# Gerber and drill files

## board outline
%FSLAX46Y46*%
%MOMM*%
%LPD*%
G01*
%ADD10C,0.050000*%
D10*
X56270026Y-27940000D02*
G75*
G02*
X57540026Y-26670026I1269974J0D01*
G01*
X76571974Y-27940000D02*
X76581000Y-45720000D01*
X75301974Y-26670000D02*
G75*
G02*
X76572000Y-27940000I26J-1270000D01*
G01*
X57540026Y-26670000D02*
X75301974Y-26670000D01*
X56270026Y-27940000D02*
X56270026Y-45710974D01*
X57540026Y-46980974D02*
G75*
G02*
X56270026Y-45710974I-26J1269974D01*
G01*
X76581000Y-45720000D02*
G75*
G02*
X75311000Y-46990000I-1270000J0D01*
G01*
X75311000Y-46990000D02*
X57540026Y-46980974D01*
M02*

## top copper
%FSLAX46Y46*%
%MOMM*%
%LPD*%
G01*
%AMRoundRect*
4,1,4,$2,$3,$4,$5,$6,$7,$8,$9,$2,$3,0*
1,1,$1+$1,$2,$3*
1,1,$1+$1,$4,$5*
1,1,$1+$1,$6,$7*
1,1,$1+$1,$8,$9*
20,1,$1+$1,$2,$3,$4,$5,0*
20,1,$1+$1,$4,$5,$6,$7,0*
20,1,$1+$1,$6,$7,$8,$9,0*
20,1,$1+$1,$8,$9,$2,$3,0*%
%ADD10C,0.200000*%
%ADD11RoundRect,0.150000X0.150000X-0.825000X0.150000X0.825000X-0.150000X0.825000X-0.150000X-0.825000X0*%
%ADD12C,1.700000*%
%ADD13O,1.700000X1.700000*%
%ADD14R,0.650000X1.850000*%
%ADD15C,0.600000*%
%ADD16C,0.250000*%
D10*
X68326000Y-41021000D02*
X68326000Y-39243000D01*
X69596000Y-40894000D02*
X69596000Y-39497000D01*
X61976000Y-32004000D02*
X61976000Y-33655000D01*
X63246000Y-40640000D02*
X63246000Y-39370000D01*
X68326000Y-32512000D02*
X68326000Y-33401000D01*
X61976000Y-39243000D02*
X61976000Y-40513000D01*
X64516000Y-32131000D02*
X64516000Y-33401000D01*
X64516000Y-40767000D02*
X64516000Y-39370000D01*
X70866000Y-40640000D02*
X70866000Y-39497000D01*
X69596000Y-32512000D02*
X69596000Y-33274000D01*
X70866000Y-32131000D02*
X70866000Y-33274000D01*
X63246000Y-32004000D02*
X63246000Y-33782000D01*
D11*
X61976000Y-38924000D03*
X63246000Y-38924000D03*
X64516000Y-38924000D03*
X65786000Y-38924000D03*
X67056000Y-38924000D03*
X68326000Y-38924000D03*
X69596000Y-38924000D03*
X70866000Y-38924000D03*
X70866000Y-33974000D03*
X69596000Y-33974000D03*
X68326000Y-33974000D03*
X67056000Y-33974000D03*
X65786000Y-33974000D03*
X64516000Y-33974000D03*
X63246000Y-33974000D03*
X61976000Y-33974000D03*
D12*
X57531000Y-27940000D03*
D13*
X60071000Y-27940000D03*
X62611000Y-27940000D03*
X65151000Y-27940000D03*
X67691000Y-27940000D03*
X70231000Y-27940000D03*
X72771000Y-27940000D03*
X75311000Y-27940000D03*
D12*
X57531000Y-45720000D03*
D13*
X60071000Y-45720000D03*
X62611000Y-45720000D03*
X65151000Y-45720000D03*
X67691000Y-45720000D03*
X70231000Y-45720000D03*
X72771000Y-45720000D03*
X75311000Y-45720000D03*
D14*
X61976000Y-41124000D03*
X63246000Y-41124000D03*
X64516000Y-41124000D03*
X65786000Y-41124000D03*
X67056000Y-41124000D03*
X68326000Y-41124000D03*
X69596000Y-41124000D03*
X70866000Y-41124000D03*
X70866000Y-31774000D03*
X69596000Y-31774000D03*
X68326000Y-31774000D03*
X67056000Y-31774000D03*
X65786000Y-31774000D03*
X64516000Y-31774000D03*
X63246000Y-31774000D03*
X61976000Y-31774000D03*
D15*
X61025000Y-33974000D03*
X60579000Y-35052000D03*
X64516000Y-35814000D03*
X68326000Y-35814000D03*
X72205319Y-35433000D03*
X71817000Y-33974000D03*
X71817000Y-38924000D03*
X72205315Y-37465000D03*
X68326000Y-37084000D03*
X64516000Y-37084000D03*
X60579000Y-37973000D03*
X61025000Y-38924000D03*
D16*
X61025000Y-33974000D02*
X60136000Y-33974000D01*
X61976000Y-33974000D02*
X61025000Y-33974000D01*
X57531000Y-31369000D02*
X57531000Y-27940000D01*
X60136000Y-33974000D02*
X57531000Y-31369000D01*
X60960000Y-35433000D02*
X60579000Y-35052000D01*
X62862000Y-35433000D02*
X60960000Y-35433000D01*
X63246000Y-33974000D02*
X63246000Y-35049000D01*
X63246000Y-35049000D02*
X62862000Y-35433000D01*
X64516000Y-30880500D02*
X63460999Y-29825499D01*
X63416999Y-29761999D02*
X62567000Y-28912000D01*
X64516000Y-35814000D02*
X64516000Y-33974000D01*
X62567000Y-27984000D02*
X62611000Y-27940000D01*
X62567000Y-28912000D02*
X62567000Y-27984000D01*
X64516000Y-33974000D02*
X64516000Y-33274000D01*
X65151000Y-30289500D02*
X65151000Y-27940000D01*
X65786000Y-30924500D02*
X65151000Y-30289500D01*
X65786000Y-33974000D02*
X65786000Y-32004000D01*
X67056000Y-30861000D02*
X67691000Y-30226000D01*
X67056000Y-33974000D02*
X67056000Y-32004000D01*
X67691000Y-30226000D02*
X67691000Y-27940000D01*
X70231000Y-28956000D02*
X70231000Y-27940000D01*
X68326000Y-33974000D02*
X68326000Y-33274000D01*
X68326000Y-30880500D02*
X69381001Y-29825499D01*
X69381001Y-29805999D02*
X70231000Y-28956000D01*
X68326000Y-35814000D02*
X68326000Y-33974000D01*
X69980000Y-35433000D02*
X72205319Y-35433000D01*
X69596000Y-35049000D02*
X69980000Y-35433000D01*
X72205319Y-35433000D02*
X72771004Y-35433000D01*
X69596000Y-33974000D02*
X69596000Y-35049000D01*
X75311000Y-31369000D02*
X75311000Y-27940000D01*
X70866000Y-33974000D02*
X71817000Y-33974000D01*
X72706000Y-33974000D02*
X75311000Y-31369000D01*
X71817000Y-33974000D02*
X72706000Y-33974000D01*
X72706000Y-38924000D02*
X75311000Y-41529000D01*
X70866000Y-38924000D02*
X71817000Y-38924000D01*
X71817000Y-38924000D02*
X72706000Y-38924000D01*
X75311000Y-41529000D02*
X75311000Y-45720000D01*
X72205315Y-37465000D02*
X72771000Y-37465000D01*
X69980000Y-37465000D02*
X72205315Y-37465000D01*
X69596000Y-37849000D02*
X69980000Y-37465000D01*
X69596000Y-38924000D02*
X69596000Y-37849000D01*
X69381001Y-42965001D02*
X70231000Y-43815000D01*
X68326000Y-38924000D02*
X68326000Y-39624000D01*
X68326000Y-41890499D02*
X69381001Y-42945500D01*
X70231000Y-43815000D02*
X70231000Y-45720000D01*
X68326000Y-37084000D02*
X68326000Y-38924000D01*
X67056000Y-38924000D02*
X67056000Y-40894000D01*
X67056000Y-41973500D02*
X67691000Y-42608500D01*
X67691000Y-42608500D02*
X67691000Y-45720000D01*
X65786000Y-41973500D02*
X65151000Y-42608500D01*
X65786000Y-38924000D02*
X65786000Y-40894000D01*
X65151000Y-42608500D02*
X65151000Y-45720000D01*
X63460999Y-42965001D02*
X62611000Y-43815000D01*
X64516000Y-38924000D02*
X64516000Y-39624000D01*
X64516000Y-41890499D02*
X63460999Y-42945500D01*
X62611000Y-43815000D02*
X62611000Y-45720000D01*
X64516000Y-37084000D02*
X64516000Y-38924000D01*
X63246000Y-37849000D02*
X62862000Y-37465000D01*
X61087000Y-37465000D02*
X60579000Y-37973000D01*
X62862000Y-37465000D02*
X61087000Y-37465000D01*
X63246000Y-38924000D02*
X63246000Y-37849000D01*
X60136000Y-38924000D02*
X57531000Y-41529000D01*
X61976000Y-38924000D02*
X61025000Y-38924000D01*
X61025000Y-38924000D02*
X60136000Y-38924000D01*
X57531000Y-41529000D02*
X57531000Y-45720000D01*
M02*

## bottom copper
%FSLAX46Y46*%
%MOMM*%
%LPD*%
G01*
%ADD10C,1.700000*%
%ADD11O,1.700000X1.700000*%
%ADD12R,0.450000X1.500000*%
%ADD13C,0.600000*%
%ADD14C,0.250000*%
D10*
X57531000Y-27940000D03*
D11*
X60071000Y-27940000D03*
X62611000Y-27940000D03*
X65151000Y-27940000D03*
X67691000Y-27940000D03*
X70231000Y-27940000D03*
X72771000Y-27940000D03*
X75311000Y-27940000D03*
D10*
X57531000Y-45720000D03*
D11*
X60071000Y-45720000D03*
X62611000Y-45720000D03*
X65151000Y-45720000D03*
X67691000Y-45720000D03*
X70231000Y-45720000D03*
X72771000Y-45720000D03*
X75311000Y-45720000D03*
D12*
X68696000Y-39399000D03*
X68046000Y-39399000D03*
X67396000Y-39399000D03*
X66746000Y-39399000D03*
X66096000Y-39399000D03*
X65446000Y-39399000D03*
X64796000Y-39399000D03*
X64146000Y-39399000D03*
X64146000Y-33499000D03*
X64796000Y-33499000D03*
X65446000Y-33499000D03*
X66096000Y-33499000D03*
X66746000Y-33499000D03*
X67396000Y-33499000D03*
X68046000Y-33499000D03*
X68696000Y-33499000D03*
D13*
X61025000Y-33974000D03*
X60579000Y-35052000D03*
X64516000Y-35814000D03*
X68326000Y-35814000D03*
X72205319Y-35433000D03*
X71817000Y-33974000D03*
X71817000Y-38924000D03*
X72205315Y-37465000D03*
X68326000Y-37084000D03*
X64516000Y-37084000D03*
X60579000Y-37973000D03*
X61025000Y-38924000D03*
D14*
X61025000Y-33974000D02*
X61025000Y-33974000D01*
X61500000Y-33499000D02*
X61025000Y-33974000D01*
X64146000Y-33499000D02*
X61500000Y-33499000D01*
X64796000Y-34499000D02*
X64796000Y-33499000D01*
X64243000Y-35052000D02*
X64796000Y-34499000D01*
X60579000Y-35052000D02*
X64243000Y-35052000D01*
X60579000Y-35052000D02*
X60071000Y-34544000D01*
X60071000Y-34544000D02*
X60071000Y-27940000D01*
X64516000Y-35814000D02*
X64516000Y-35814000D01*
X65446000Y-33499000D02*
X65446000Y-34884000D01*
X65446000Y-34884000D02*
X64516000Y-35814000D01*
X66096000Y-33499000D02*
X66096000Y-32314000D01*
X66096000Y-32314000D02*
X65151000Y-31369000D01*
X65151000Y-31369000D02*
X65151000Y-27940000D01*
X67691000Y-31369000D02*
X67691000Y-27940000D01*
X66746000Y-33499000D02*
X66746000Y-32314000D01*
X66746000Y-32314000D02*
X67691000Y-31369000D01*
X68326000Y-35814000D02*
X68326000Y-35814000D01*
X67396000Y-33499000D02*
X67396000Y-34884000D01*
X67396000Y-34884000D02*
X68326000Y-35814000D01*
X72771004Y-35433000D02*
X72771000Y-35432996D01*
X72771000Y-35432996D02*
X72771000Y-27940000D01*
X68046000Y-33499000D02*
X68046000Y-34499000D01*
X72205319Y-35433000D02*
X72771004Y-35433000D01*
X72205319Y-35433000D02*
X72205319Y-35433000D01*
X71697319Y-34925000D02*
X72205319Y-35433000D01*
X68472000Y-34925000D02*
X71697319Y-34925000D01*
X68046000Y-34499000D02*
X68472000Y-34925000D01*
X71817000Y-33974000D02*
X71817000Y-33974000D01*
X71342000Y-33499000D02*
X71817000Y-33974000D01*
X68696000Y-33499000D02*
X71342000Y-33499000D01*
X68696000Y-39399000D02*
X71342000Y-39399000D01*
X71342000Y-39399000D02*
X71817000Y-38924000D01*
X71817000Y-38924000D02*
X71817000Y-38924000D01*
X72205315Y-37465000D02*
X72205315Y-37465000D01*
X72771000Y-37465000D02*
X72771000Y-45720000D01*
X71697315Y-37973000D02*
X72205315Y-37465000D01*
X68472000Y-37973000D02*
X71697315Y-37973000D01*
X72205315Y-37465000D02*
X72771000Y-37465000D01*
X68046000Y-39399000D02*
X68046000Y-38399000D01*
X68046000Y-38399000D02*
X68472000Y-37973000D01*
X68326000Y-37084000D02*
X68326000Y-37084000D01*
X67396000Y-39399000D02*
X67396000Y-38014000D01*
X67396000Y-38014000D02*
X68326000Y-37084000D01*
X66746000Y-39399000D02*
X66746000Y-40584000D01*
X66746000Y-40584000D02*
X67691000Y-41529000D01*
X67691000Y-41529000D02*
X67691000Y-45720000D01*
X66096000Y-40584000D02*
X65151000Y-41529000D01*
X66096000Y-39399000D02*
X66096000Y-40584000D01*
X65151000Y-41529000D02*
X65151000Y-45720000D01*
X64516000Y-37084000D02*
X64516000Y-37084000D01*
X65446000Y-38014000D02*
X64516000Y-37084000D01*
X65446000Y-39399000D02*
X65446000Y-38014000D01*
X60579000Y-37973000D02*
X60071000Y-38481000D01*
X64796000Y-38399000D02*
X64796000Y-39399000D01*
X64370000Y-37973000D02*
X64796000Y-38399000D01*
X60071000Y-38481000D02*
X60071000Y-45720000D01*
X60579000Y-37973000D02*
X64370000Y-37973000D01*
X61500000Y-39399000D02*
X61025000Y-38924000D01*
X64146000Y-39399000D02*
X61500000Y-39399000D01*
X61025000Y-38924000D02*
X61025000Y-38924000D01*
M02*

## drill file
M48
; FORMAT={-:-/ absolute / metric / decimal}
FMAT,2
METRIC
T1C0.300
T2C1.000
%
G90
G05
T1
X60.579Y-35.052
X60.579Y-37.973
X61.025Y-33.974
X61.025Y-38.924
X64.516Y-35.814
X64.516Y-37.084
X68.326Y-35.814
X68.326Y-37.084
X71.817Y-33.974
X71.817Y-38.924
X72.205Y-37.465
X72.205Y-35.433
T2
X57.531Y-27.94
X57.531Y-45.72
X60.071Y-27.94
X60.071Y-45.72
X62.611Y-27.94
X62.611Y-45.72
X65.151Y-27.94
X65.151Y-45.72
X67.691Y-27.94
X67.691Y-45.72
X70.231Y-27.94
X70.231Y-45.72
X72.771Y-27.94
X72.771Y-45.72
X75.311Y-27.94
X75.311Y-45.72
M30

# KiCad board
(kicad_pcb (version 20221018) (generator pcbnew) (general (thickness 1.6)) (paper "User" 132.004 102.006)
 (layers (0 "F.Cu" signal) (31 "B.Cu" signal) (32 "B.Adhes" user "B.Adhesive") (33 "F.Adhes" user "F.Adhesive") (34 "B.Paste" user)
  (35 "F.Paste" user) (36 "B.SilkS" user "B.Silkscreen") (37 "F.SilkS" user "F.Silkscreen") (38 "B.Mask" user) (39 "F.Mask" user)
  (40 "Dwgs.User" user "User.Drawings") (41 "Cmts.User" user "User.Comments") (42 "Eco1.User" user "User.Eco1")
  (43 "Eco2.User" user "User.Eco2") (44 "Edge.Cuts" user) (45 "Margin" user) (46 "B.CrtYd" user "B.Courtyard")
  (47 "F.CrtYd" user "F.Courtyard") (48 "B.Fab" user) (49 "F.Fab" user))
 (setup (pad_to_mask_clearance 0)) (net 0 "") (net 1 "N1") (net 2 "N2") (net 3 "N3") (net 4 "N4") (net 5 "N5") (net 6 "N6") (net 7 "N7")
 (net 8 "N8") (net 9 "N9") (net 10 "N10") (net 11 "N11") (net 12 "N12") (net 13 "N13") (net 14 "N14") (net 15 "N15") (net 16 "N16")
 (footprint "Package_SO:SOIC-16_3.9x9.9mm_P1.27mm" (layer "F.Cu") (at 66.421 36.449 90)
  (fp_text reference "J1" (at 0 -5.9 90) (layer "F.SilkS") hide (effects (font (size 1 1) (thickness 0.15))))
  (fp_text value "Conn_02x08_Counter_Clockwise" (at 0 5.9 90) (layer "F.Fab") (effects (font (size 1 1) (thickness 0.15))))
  (pad "1" smd roundrect (at -2.475 -4.445 90) (size 1.95 0.6) (layers "F.Cu" "F.Paste" "F.Mask") (roundrect_rratio 0.25) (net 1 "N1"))
  (pad "2" smd roundrect (at -2.475 -3.175 90) (size 1.95 0.6) (layers "F.Cu" "F.Paste" "F.Mask") (roundrect_rratio 0.25) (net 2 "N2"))
  (pad "3" smd roundrect (at -2.475 -1.905 90) (size 1.95 0.6) (layers "F.Cu" "F.Paste" "F.Mask") (roundrect_rratio 0.25) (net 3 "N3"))
  (pad "4" smd roundrect (at -2.475 -0.635 90) (size 1.95 0.6) (layers "F.Cu" "F.Paste" "F.Mask") (roundrect_rratio 0.25) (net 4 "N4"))
  (pad "5" smd roundrect (at -2.475 0.635 90) (size 1.95 0.6) (layers "F.Cu" "F.Paste" "F.Mask") (roundrect_rratio 0.25) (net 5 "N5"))
  (pad "6" smd roundrect (at -2.475 1.905 90) (size 1.95 0.6) (layers "F.Cu" "F.Paste" "F.Mask") (roundrect_rratio 0.25) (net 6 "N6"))
  (pad "7" smd roundrect (at -2.475 3.175 90) (size 1.95 0.6) (layers "F.Cu" "F.Paste" "F.Mask") (roundrect_rratio 0.25) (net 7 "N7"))
  (pad "8" smd roundrect (at -2.475 4.445 90) (size 1.95 0.6) (layers "F.Cu" "F.Paste" "F.Mask") (roundrect_rratio 0.25) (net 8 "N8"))
  (pad "9" smd roundrect (at 2.475 4.445 90) (size 1.95 0.6) (layers "F.Cu" "F.Paste" "F.Mask") (roundrect_rratio 0.25) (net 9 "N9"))
  (pad "10" smd roundrect (at 2.475 3.175 90) (size 1.95 0.6) (layers "F.Cu" "F.Paste" "F.Mask") (roundrect_rratio 0.25) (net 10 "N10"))
  (pad "11" smd roundrect (at 2.475 1.905 90) (size 1.95 0.6) (layers "F.Cu" "F.Paste" "F.Mask") (roundrect_rratio 0.25) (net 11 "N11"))
  (pad "12" smd roundrect (at 2.475 0.635 90) (size 1.95 0.6) (layers "F.Cu" "F.Paste" "F.Mask") (roundrect_rratio 0.25) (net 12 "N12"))
  (pad "13" smd roundrect (at 2.475 -0.635 90) (size 1.95 0.6) (layers "F.Cu" "F.Paste" "F.Mask") (roundrect_rratio 0.25) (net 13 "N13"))
  (pad "14" smd roundrect (at 2.475 -1.905 90) (size 1.95 0.6) (layers "F.Cu" "F.Paste" "F.Mask") (roundrect_rratio 0.25) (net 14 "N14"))
  (pad "15" smd roundrect (at 2.475 -3.175 90) (size 1.95 0.6) (layers "F.Cu" "F.Paste" "F.Mask") (roundrect_rratio 0.25) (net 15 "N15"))
  (pad "16" smd roundrect (at 2.475 -4.445 90) (size 1.95 0.6) (layers "F.Cu" "F.Paste" "F.Mask") (roundrect_rratio 0.25) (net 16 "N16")))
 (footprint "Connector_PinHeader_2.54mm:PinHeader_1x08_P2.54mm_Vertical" (layer "F.Cu") (at 57.531 27.94 90)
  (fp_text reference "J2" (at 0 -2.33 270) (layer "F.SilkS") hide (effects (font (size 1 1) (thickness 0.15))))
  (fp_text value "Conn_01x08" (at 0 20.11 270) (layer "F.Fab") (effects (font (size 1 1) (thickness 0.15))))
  (pad "1" thru_hole circle (at 0 0 90) (size 1.7 1.7) (drill 1) (layers "*.Cu" "*.Mask") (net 16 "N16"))
  (pad "2" thru_hole oval (at 0 2.54 90) (size 1.7 1.7) (drill 1) (layers "*.Cu" "*.Mask") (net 15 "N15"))
  (pad "3" thru_hole oval (at 0 5.08 90) (size 1.7 1.7) (drill 1) (layers "*.Cu" "*.Mask") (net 14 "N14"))
  (pad "4" thru_hole oval (at 0 7.62 90) (size 1.7 1.7) (drill 1) (layers "*.Cu" "*.Mask") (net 13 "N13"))
  (pad "5" thru_hole oval (at 0 10.16 90) (size 1.7 1.7) (drill 1) (layers "*.Cu" "*.Mask") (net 12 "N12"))
  (pad "6" thru_hole oval (at 0 12.7 90) (size 1.7 1.7) (drill 1) (layers "*.Cu" "*.Mask") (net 11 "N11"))
  (pad "7" thru_hole oval (at 0 15.24 90) (size 1.7 1.7) (drill 1) (layers "*.Cu" "*.Mask") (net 10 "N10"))
  (pad "8" thru_hole oval (at 0 17.78 90) (size 1.7 1.7) (drill 1) (layers "*.Cu" "*.Mask") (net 9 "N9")))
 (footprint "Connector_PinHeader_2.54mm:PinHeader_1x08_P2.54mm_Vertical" (layer "F.Cu") (at 57.531 45.72 90)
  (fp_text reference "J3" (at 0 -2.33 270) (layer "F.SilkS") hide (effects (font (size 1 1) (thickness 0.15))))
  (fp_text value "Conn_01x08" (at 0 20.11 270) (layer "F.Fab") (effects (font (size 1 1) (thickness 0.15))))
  (pad "1" thru_hole circle (at 0 0 90) (size 1.7 1.7) (drill 1) (layers "*.Cu" "*.Mask") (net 1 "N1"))
  (pad "2" thru_hole oval (at 0 2.54 90) (size 1.7 1.7) (drill 1) (layers "*.Cu" "*.Mask") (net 2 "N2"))
  (pad "3" thru_hole oval (at 0 5.08 90) (size 1.7 1.7) (drill 1) (layers "*.Cu" "*.Mask") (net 3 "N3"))
  (pad "4" thru_hole oval (at 0 7.62 90) (size 1.7 1.7) (drill 1) (layers "*.Cu" "*.Mask") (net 4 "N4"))
  (pad "5" thru_hole oval (at 0 10.16 90) (size 1.7 1.7) (drill 1) (layers "*.Cu" "*.Mask") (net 5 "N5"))
  (pad "6" thru_hole oval (at 0 12.7 90) (size 1.7 1.7) (drill 1) (layers "*.Cu" "*.Mask") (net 6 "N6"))
  (pad "7" thru_hole oval (at 0 15.24 90) (size 1.7 1.7) (drill 1) (layers "*.Cu" "*.Mask") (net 7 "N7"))
  (pad "8" thru_hole oval (at 0 17.78 90) (size 1.7 1.7) (drill 1) (layers "*.Cu" "*.Mask") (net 8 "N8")))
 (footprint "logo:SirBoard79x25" (layer "F.Cu") (at 66.421 36.449)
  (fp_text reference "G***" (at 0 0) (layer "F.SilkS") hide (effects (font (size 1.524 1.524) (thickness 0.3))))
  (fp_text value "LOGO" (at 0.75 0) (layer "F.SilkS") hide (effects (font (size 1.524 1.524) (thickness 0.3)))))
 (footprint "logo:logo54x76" (layer "F.Cu") (at 58.801 36.449)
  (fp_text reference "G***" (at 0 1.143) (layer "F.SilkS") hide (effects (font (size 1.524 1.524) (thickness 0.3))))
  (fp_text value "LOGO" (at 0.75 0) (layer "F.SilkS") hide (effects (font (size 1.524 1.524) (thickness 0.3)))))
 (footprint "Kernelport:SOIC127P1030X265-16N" (layer "F.Cu") (at 66.421 36.449 90)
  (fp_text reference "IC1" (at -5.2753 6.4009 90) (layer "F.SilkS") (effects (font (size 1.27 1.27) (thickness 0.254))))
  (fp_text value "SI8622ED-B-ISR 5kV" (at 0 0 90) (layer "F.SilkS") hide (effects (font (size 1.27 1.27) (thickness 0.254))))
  (pad "1" smd rect (at -4.675 -4.445 180) (size 0.65 1.85) (layers "F.Cu" "F.Paste" "F.Mask"))
  (pad "2" smd rect (at -4.675 -3.175 180) (size 0.65 1.85) (layers "F.Cu" "F.Paste" "F.Mask"))
  (pad "3" smd rect (at -4.675 -1.905 180) (size 0.65 1.85) (layers "F.Cu" "F.Paste" "F.Mask"))
  (pad "4" smd rect (at -4.675 -0.635 180) (size 0.65 1.85) (layers "F.Cu" "F.Paste" "F.Mask"))
  (pad "5" smd rect (at -4.675 0.635 180) (size 0.65 1.85) (layers "F.Cu" "F.Paste" "F.Mask"))
  (pad "6" smd rect (at -4.675 1.905 180) (size 0.65 1.85) (layers "F.Cu" "F.Paste" "F.Mask"))
  (pad "7" smd rect (at -4.675 3.175 180) (size 0.65 1.85) (layers "F.Cu" "F.Paste" "F.Mask"))
  (pad "8" smd rect (at -4.675 4.445 180) (size 0.65 1.85) (layers "F.Cu" "F.Paste" "F.Mask"))
  (pad "9" smd rect (at 4.675 4.445 180) (size 0.65 1.85) (layers "F.Cu" "F.Paste" "F.Mask"))
  (pad "10" smd rect (at 4.675 3.175 180) (size 0.65 1.85) (layers "F.Cu" "F.Paste" "F.Mask"))
  (pad "11" smd rect (at 4.675 1.905 180) (size 0.65 1.85) (layers "F.Cu" "F.Paste" "F.Mask"))
  (pad "12" smd rect (at 4.675 0.635 180) (size 0.65 1.85) (layers "F.Cu" "F.Paste" "F.Mask"))
  (pad "13" smd rect (at 4.675 -0.635 180) (size 0.65 1.85) (layers "F.Cu" "F.Paste" "F.Mask"))
  (pad "14" smd rect (at 4.675 -1.905 180) (size 0.65 1.85) (layers "F.Cu" "F.Paste" "F.Mask"))
  (pad "15" smd rect (at 4.675 -3.175 180) (size 0.65 1.85) (layers "F.Cu" "F.Paste" "F.Mask"))
  (pad "16" smd rect (at 4.675 -4.445 180) (size 0.65 1.85) (layers "F.Cu" "F.Paste" "F.Mask")))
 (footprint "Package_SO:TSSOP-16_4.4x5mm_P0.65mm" (layer "B.Cu") (at 66.421 36.449 90)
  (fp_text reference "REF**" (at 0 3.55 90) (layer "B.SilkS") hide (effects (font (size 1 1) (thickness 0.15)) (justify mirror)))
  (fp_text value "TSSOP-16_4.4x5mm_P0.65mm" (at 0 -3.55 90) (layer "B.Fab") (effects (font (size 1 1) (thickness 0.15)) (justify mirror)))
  (pad "1" smd rect (at -2.95 2.275 90) (size 1.5 0.45) (layers "B.Cu" "B.Paste" "B.Mask") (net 8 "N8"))
  (pad "2" smd rect (at -2.95 1.625 90) (size 1.5 0.45) (layers "B.Cu" "B.Paste" "B.Mask") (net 7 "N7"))
  (pad "3" smd rect (at -2.95 0.975 90) (size 1.5 0.45) (layers "B.Cu" "B.Paste" "B.Mask") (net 6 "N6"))
  (pad "4" smd rect (at -2.95 0.325 90) (size 1.5 0.45) (layers "B.Cu" "B.Paste" "B.Mask") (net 5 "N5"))
  (pad "5" smd rect (at -2.95 -0.325 90) (size 1.5 0.45) (layers "B.Cu" "B.Paste" "B.Mask") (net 4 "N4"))
  (pad "6" smd rect (at -2.95 -0.975 90) (size 1.5 0.45) (layers "B.Cu" "B.Paste" "B.Mask") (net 3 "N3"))
  (pad "7" smd rect (at -2.95 -1.625 90) (size 1.5 0.45) (layers "B.Cu" "B.Paste" "B.Mask") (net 2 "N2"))
  (pad "8" smd rect (at -2.95 -2.275 90) (size 1.5 0.45) (layers "B.Cu" "B.Paste" "B.Mask") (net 1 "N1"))
  (pad "9" smd rect (at 2.95 -2.275 90) (size 1.5 0.45) (layers "B.Cu" "B.Paste" "B.Mask") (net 16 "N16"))
  (pad "10" smd rect (at 2.95 -1.625 90) (size 1.5 0.45) (layers "B.Cu" "B.Paste" "B.Mask") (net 15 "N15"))
  (pad "11" smd rect (at 2.95 -0.975 90) (size 1.5 0.45) (layers "B.Cu" "B.Paste" "B.Mask") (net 14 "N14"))
  (pad "12" smd rect (at 2.95 -0.325 90) (size 1.5 0.45) (layers "B.Cu" "B.Paste" "B.Mask") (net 13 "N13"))
  (pad "13" smd rect (at 2.95 0.325 90) (size 1.5 0.45) (layers "B.Cu" "B.Paste" "B.Mask") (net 12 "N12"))
  (pad "14" smd rect (at 2.95 0.975 90) (size 1.5 0.45) (layers "B.Cu" "B.Paste" "B.Mask") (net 11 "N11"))
  (pad "15" smd rect (at 2.95 1.625 90) (size 1.5 0.45) (layers "B.Cu" "B.Paste" "B.Mask") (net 10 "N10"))
  (pad "16" smd rect (at 2.95 2.275 90) (size 1.5 0.45) (layers "B.Cu" "B.Paste" "B.Mask") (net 9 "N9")))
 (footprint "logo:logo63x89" (layer "B.Cu") (at 72.771 36.449 180)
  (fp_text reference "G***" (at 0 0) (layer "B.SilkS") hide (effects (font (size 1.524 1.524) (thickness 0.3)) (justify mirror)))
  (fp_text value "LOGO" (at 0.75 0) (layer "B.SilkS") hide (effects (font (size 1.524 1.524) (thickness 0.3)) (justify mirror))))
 (gr_line (start 68.326 41.021) (end 68.326 39.243) (stroke (width 0.2) (type default)) (layer "F.Cu"))
 (gr_line (start 69.596 40.894) (end 69.596 39.497) (stroke (width 0.2) (type default)) (layer "F.Cu"))
 (gr_line (start 61.976 32.004) (end 61.976 33.655) (stroke (width 0.2) (type default)) (layer "F.Cu"))
 (gr_line (start 63.246 40.64) (end 63.246 39.37) (stroke (width 0.2) (type default)) (layer "F.Cu"))
 (gr_line (start 68.326 32.512) (end 68.326 33.401) (stroke (width 0.2) (type default)) (layer "F.Cu"))
 (gr_line (start 61.976 39.243) (end 61.976 40.513) (stroke (width 0.2) (type default)) (layer "F.Cu"))
 (gr_line (start 64.516 32.131) (end 64.516 33.401) (stroke (width 0.2) (type default)) (layer "F.Cu"))
 (gr_line (start 64.516 40.767) (end 64.516 39.37) (stroke (width 0.2) (type default)) (layer "F.Cu"))
 (gr_line (start 70.866 40.64) (end 70.866 39.497) (stroke (width 0.2) (type default)) (layer "F.Cu"))
 (gr_line (start 69.596 32.512) (end 69.596 33.274) (stroke (width 0.2) (type default)) (layer "F.Cu"))
 (gr_line (start 70.866 32.131) (end 70.866 33.274) (stroke (width 0.2) (type default)) (layer "F.Cu"))
 (gr_line (start 63.246 32.004) (end 63.246 33.782) (stroke (width 0.2) (type default)) (layer "F.Cu"))
 (gr_arc (start 56.270026 27.94) (mid 56.642 27.041974) (end 57.540026 26.67) (stroke (width 0.05) (type default)) (layer "Edge.Cuts"))
 (gr_line (start 76.571974 27.94) (end 76.581 45.72) (stroke (width 0.05) (type default)) (layer "Edge.Cuts"))
 (gr_arc (start 75.301974 26.67) (mid 76.2 27.041974) (end 76.571974 27.94) (stroke (width 0.05) (type default)) (layer "Edge.Cuts"))
 (gr_line (start 57.540026 26.67) (end 75.301974 26.67) (stroke (width 0.05) (type default)) (layer "Edge.Cuts"))
 (gr_line (start 56.270026 27.94) (end 56.270026 45.710974) (stroke (width 0.05) (type default)) (layer "Edge.Cuts"))
 (gr_arc (start 57.540026 46.980974) (mid 56.642 46.609) (end 56.270026 45.710974) (stroke (width 0.05) (type default)) (layer "Edge.Cuts"))
 (gr_arc (start 76.581 45.72) (mid 76.209026 46.618026) (end 75.311 46.99) (stroke (width 0.05) (type default)) (layer "Edge.Cuts"))
 (gr_line (start 75.311 46.99) (end 57.540026 46.980974) (stroke (width 0.05) (type default)) (layer "Edge.Cuts"))
 (segment (start 61.025 33.974) (end 60.136 33.974) (width 0.25) (layer "F.Cu") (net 16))
 (segment (start 61.976 33.974) (end 61.025 33.974) (width 0.25) (layer "F.Cu") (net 16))
 (segment (start 57.531 31.369) (end 57.531 27.94) (width 0.25) (layer "F.Cu") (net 16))
 (segment (start 60.136 33.974) (end 57.531 31.369) (width 0.25) (layer "F.Cu") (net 16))
 (via (at 61.025 33.974) (size 0.6) (drill 0.3) (layers "F.Cu" "B.Cu") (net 16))
 (segment (start 61.025 33.974) (end 61.025 33.974) (width 0.25) (layer "B.Cu") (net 16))
 (segment (start 61.5 33.499) (end 61.025 33.974) (width 0.25) (layer "B.Cu") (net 16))
 (segment (start 64.146 33.499) (end 61.5 33.499) (width 0.25) (layer "B.Cu") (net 16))
 (segment (start 60.96 35.433) (end 60.579 35.052) (width 0.25) (layer "F.Cu") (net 15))
 (segment (start 62.862 35.433) (end 60.96 35.433) (width 0.25) (layer "F.Cu") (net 15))
 (segment (start 63.246 33.974) (end 63.246 35.049) (width 0.25) (layer "F.Cu") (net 15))
 (segment (start 63.246 35.049) (end 62.862 35.433) (width 0.25) (layer "F.Cu") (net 15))
 (via (at 60.579 35.052) (size 0.6) (drill 0.3) (layers "F.Cu" "B.Cu") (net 15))
 (segment (start 64.796 34.499) (end 64.796 33.499) (width 0.25) (layer "B.Cu") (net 15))
 (segment (start 64.243 35.052) (end 64.796 34.499) (width 0.25) (layer "B.Cu") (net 15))
 (segment (start 60.579 35.052) (end 64.243 35.052) (width 0.25) (layer "B.Cu") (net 15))
 (segment (start 60.579 35.052) (end 60.071 34.544) (width 0.25) (layer "B.Cu") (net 15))
 (segment (start 60.071 34.544) (end 60.071 27.94) (width 0.25) (layer "B.Cu") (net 15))
 (segment (start 64.516 30.8805) (end 63.460999 29.825499) (width 0.25) (layer "F.Cu") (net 14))
 (segment (start 63.416999 29.761999) (end 62.567 28.912) (width 0.25) (layer "F.Cu") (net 14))
 (segment (start 64.516 35.814) (end 64.516 33.974) (width 0.25) (layer "F.Cu") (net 14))
 (segment (start 62.567 27.984) (end 62.611 27.94) (width 0.25) (layer "F.Cu") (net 14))
 (segment (start 62.567 28.912) (end 62.567 27.984) (width 0.25) (layer "F.Cu") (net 14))
 (segment (start 64.516 33.974) (end 64.516 33.274) (width 0.25) (layer "F.Cu") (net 14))
 (via (at 64.516 35.814) (size 0.6) (drill 0.3) (layers "F.Cu" "B.Cu") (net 14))
 (segment (start 64.516 35.814) (end 64.516 35.814) (width 0.25) (layer "B.Cu") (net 14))
 (segment (start 65.446 33.499) (end 65.446 34.884) (width 0.25) (layer "B.Cu") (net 14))
 (segment (start 65.446 34.884) (end 64.516 35.814) (width 0.25) (layer "B.Cu") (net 14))
 (segment (start 65.151 30.2895) (end 65.151 27.94) (width 0.25) (layer "F.Cu") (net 13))
 (segment (start 65.786 30.9245) (end 65.151 30.2895) (width 0.25) (layer "F.Cu") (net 13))
 (segment (start 65.786 33.974) (end 65.786 32.004) (width 0.25) (layer "F.Cu") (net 13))
 (segment (start 66.096 33.499) (end 66.096 32.314) (width 0.25) (layer "B.Cu") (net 13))
 (segment (start 66.096 32.314) (end 65.151 31.369) (width 0.25) (layer "B.Cu") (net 13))
 (segment (start 65.151 31.369) (end 65.151 27.94) (width 0.25) (layer "B.Cu") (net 13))
 (segment (start 67.056 30.861) (end 67.691 30.226) (width 0.25) (layer "F.Cu") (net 12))
 (segment (start 67.056 33.974) (end 67.056 32.004) (width 0.25) (layer "F.Cu") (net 12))
 (segment (start 67.691 30.226) (end 67.691 27.94) (width 0.25) (layer "F.Cu") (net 12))
 (segment (start 67.691 31.369) (end 67.691 27.94) (width 0.25) (layer "B.Cu") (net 12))
 (segment (start 66.746 33.499) (end 66.746 32.314) (width 0.25) (layer "B.Cu") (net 12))
 (segment (start 66.746 32.314) (end 67.691 31.369) (width 0.25) (layer "B.Cu") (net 12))
 (segment (start 70.231 28.956) (end 70.231 27.94) (width 0.25) (layer "F.Cu") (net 11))
 (segment (start 68.326 33.974) (end 68.326 33.274) (width 0.25) (layer "F.Cu") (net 11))
 (segment (start 68.326 30.8805) (end 69.381001 29.825499) (width 0.25) (layer "F.Cu") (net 11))
 (segment (start 69.381001 29.805999) (end 70.231 28.956) (width 0.25) (layer "F.Cu") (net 11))
 (segment (start 68.326 35.814) (end 68.326 33.974) (width 0.25) (layer "F.Cu") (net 11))
 (via (at 68.326 35.814) (size 0.6) (drill 0.3) (layers "F.Cu" "B.Cu") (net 11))
 (segment (start 68.326 35.814) (end 68.326 35.814) (width 0.25) (layer "B.Cu") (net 11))
 (segment (start 67.396 33.499) (end 67.396 34.884) (width 0.25) (layer "B.Cu") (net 11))
 (segment (start 67.396 34.884) (end 68.326 35.814) (width 0.25) (layer "B.Cu") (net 11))
 (segment (start 69.98 35.433) (end 72.205319 35.433) (width 0.25) (layer "F.Cu") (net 10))
 (segment (start 69.596 35.049) (end 69.98 35.433) (width 0.25) (layer "F.Cu") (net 10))
 (segment (start 72.205319 35.433) (end 72.771004 35.433) (width 0.25) (layer "F.Cu") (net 10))
 (segment (start 69.596 33.974) (end 69.596 35.049) (width 0.25) (layer "F.Cu") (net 10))
 (via (at 72.205319 35.433) (size 0.6) (drill 0.3) (layers "F.Cu" "B.Cu") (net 10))
 (segment (start 72.771004 35.433) (end 72.771 35.432996) (width 0.25) (layer "B.Cu") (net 10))
 (segment (start 72.771 35.432996) (end 72.771 27.94) (width 0.25) (layer "B.Cu") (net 10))
 (segment (start 68.046 33.499) (end 68.046 34.499) (width 0.25) (layer "B.Cu") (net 10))
 (segment (start 72.205319 35.433) (end 72.771004 35.433) (width 0.25) (layer "B.Cu") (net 10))
 (segment (start 72.205319 35.433) (end 72.205319 35.433) (width 0.25) (layer "B.Cu") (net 10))
 (segment (start 71.697319 34.925) (end 72.205319 35.433) (width 0.25) (layer "B.Cu") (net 10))
 (segment (start 68.472 34.925) (end 71.697319 34.925) (width 0.25) (layer "B.Cu") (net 10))
 (segment (start 68.046 34.499) (end 68.472 34.925) (width 0.25) (layer "B.Cu") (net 10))
 (segment (start 75.311 31.369) (end 75.311 27.94) (width 0.25) (layer "F.Cu") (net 9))
 (segment (start 70.866 33.974) (end 71.817 33.974) (width 0.25) (layer "F.Cu") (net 9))
 (segment (start 72.706 33.974) (end 75.311 31.369) (width 0.25) (layer "F.Cu") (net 9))
 (segment (start 71.817 33.974) (end 72.706 33.974) (width 0.25) (layer "F.Cu") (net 9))
 (via (at 71.817 33.974) (size 0.6) (drill 0.3) (layers "F.Cu" "B.Cu") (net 9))
 (segment (start 71.817 33.974) (end 71.817 33.974) (width 0.25) (layer "B.Cu") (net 9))
 (segment (start 71.342 33.499) (end 71.817 33.974) (width 0.25) (layer "B.Cu") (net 9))
 (segment (start 68.696 33.499) (end 71.342 33.499) (width 0.25) (layer "B.Cu") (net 9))
 (segment (start 72.706 38.924) (end 75.311 41.529) (width 0.25) (layer "F.Cu") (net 8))
 (segment (start 70.866 38.924) (end 71.817 38.924) (width 0.25) (layer "F.Cu") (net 8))
 (segment (start 71.817 38.924) (end 72.706 38.924) (width 0.25) (layer "F.Cu") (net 8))
 (segment (start 75.311 41.529) (end 75.311 45.72) (width 0.25) (layer "F.Cu") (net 8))
 (via (at 71.817 38.924) (size 0.6) (drill 0.3) (layers "F.Cu" "B.Cu") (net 8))
 (segment (start 68.696 39.399) (end 71.342 39.399) (width 0.25) (layer "B.Cu") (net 8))
 (segment (start 71.342 39.399) (end 71.817 38.924) (width 0.25) (layer "B.Cu") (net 8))
 (segment (start 71.817 38.924) (end 71.817 38.924) (width 0.25) (layer "B.Cu") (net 8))
 (segment (start 72.205315 37.465) (end 72.771 37.465) (width 0.25) (layer "F.Cu") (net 7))
 (segment (start 69.98 37.465) (end 72.205315 37.465) (width 0.25) (layer "F.Cu") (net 7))
 (segment (start 69.596 37.849) (end 69.98 37.465) (width 0.25) (layer "F.Cu") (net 7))
 (segment (start 69.596 38.924) (end 69.596 37.849) (width 0.25) (layer "F.Cu") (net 7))
 (via (at 72.205315 37.465) (size 0.6) (drill 0.3) (layers "F.Cu" "B.Cu") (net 7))
 (segment (start 72.205315 37.465) (end 72.205315 37.465) (width 0.25) (layer "B.Cu") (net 7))
 (segment (start 72.771 37.465) (end 72.771 45.72) (width 0.25) (layer "B.Cu") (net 7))
 (segment (start 71.697315 37.973) (end 72.205315 37.465) (width 0.25) (layer "B.Cu") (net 7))
 (segment (start 68.472 37.973) (end 71.697315 37.973) (width 0.25) (layer "B.Cu") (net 7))
 (segment (start 72.205315 37.465) (end 72.771 37.465) (width 0.25) (layer "B.Cu") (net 7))
 (segment (start 68.046 39.399) (end 68.046 38.399) (width 0.25) (layer "B.Cu") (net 7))
 (segment (start 68.046 38.399) (end 68.472 37.973) (width 0.25) (layer "B.Cu") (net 7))
 (segment (start 69.381001 42.965001) (end 70.231 43.815) (width 0.25) (layer "F.Cu") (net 6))
 (segment (start 68.326 38.924) (end 68.326 39.624) (width 0.25) (layer "F.Cu") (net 6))
 (segment (start 68.326 41.890499) (end 69.381001 42.9455) (width 0.25) (layer "F.Cu") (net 6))
 (segment (start 70.231 43.815) (end 70.231 45.72) (width 0.25) (layer "F.Cu") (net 6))
 (segment (start 68.326 37.084) (end 68.326 38.924) (width 0.25) (layer "F.Cu") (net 6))
 (via (at 68.326 37.084) (size 0.6) (drill 0.3) (layers "F.Cu" "B.Cu") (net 6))
 (segment (start 68.326 37.084) (end 68.326 37.084) (width 0.25) (layer "B.Cu") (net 6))
 (segment (start 67.396 39.399) (end 67.396 38.014) (width 0.25) (layer "B.Cu") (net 6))
 (segment (start 67.396 38.014) (end 68.326 37.084) (width 0.25) (layer "B.Cu") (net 6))
 (segment (start 67.056 38.924) (end 67.056 40.894) (width 0.25) (layer "F.Cu") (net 5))
 (segment (start 67.056 41.9735) (end 67.691 42.6085) (width 0.25) (layer "F.Cu") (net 5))
 (segment (start 67.691 42.6085) (end 67.691 45.72) (width 0.25) (layer "F.Cu") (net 5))
 (segment (start 66.746 39.399) (end 66.746 40.584) (width 0.25) (layer "B.Cu") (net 5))
 (segment (start 66.746 40.584) (end 67.691 41.529) (width 0.25) (layer "B.Cu") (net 5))
 (segment (start 67.691 41.529) (end 67.691 45.72) (width 0.25) (layer "B.Cu") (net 5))
 (segment (start 65.786 41.9735) (end 65.151 42.6085) (width 0.25) (layer "F.Cu") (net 4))
 (segment (start 65.786 38.924) (end 65.786 40.894) (width 0.25) (layer "F.Cu") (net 4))
 (segment (start 65.151 42.6085) (end 65.151 45.72) (width 0.25) (layer "F.Cu") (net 4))
 (segment (start 66.096 40.584) (end 65.151 41.529) (width 0.25) (layer "B.Cu") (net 4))
 (segment (start 66.096 39.399) (end 66.096 40.584) (width 0.25) (layer "B.Cu") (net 4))
 (segment (start 65.151 41.529) (end 65.151 45.72) (width 0.25) (layer "B.Cu") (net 4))
 (segment (start 63.460999 42.965001) (end 62.611 43.815) (width 0.25) (layer "F.Cu") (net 3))
 (segment (start 64.516 38.924) (end 64.516 39.624) (width 0.25) (layer "F.Cu") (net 3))
 (segment (start 64.516 41.890499) (end 63.460999 42.9455) (width 0.25) (layer "F.Cu") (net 3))
 (segment (start 62.611 43.815) (end 62.611 45.72) (width 0.25) (layer "F.Cu") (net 3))
 (segment (start 64.516 37.084) (end 64.516 38.924) (width 0.25) (layer "F.Cu") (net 3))
 (via (at 64.516 37.084) (size 0.6) (drill 0.3) (layers "F.Cu" "B.Cu") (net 3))
 (segment (start 64.516 37.084) (end 64.516 37.084) (width 0.25) (layer "B.Cu") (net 3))
 (segment (start 65.446 38.014) (end 64.516 37.084) (width 0.25) (layer "B.Cu") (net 3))
 (segment (start 65.446 39.399) (end 65.446 38.014) (width 0.25) (layer "B.Cu") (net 3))
 (segment (start 63.246 37.849) (end 62.862 37.465) (width 0.25) (layer "F.Cu") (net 2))
 (segment (start 61.087 37.465) (end 60.579 37.973) (width 0.25) (layer "F.Cu") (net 2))
 (segment (start 62.862 37.465) (end 61.087 37.465) (width 0.25) (layer "F.Cu") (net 2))
 (segment (start 63.246 38.924) (end 63.246 37.849) (width 0.25) (layer "F.Cu") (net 2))
 (via (at 60.579 37.973) (size 0.6) (drill 0.3) (layers "F.Cu" "B.Cu") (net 2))
 (segment (start 60.579 37.973) (end 60.071 38.481) (width 0.25) (layer "B.Cu") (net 2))
 (segment (start 64.796 38.399) (end 64.796 39.399) (width 0.25) (layer "B.Cu") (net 2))
 (segment (start 64.37 37.973) (end 64.796 38.399) (width 0.25) (layer "B.Cu") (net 2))
 (segment (start 60.071 38.481) (end 60.071 45.72) (width 0.25) (layer "B.Cu") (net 2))
 (segment (start 60.579 37.973) (end 64.37 37.973) (width 0.25) (layer "B.Cu") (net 2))
 (segment (start 60.136 38.924) (end 57.531 41.529) (width 0.25) (layer "F.Cu") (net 1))
 (segment (start 61.976 38.924) (end 61.025 38.924) (width 0.25) (layer "F.Cu") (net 1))
 (segment (start 61.025 38.924) (end 60.136 38.924) (width 0.25) (layer "F.Cu") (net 1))
 (segment (start 57.531 41.529) (end 57.531 45.72) (width 0.25) (layer "F.Cu") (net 1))
 (via (at 61.025 38.924) (size 0.6) (drill 0.3) (layers "F.Cu" "B.Cu") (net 1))
 (segment (start 61.5 39.399) (end 61.025 38.924) (width 0.25) (layer "B.Cu") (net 1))
 (segment (start 64.146 39.399) (end 61.5 39.399) (width 0.25) (layer "B.Cu") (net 1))
 (segment (start 61.025 38.924) (end 61.025 38.924) (width 0.25) (layer "B.Cu") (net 1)))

